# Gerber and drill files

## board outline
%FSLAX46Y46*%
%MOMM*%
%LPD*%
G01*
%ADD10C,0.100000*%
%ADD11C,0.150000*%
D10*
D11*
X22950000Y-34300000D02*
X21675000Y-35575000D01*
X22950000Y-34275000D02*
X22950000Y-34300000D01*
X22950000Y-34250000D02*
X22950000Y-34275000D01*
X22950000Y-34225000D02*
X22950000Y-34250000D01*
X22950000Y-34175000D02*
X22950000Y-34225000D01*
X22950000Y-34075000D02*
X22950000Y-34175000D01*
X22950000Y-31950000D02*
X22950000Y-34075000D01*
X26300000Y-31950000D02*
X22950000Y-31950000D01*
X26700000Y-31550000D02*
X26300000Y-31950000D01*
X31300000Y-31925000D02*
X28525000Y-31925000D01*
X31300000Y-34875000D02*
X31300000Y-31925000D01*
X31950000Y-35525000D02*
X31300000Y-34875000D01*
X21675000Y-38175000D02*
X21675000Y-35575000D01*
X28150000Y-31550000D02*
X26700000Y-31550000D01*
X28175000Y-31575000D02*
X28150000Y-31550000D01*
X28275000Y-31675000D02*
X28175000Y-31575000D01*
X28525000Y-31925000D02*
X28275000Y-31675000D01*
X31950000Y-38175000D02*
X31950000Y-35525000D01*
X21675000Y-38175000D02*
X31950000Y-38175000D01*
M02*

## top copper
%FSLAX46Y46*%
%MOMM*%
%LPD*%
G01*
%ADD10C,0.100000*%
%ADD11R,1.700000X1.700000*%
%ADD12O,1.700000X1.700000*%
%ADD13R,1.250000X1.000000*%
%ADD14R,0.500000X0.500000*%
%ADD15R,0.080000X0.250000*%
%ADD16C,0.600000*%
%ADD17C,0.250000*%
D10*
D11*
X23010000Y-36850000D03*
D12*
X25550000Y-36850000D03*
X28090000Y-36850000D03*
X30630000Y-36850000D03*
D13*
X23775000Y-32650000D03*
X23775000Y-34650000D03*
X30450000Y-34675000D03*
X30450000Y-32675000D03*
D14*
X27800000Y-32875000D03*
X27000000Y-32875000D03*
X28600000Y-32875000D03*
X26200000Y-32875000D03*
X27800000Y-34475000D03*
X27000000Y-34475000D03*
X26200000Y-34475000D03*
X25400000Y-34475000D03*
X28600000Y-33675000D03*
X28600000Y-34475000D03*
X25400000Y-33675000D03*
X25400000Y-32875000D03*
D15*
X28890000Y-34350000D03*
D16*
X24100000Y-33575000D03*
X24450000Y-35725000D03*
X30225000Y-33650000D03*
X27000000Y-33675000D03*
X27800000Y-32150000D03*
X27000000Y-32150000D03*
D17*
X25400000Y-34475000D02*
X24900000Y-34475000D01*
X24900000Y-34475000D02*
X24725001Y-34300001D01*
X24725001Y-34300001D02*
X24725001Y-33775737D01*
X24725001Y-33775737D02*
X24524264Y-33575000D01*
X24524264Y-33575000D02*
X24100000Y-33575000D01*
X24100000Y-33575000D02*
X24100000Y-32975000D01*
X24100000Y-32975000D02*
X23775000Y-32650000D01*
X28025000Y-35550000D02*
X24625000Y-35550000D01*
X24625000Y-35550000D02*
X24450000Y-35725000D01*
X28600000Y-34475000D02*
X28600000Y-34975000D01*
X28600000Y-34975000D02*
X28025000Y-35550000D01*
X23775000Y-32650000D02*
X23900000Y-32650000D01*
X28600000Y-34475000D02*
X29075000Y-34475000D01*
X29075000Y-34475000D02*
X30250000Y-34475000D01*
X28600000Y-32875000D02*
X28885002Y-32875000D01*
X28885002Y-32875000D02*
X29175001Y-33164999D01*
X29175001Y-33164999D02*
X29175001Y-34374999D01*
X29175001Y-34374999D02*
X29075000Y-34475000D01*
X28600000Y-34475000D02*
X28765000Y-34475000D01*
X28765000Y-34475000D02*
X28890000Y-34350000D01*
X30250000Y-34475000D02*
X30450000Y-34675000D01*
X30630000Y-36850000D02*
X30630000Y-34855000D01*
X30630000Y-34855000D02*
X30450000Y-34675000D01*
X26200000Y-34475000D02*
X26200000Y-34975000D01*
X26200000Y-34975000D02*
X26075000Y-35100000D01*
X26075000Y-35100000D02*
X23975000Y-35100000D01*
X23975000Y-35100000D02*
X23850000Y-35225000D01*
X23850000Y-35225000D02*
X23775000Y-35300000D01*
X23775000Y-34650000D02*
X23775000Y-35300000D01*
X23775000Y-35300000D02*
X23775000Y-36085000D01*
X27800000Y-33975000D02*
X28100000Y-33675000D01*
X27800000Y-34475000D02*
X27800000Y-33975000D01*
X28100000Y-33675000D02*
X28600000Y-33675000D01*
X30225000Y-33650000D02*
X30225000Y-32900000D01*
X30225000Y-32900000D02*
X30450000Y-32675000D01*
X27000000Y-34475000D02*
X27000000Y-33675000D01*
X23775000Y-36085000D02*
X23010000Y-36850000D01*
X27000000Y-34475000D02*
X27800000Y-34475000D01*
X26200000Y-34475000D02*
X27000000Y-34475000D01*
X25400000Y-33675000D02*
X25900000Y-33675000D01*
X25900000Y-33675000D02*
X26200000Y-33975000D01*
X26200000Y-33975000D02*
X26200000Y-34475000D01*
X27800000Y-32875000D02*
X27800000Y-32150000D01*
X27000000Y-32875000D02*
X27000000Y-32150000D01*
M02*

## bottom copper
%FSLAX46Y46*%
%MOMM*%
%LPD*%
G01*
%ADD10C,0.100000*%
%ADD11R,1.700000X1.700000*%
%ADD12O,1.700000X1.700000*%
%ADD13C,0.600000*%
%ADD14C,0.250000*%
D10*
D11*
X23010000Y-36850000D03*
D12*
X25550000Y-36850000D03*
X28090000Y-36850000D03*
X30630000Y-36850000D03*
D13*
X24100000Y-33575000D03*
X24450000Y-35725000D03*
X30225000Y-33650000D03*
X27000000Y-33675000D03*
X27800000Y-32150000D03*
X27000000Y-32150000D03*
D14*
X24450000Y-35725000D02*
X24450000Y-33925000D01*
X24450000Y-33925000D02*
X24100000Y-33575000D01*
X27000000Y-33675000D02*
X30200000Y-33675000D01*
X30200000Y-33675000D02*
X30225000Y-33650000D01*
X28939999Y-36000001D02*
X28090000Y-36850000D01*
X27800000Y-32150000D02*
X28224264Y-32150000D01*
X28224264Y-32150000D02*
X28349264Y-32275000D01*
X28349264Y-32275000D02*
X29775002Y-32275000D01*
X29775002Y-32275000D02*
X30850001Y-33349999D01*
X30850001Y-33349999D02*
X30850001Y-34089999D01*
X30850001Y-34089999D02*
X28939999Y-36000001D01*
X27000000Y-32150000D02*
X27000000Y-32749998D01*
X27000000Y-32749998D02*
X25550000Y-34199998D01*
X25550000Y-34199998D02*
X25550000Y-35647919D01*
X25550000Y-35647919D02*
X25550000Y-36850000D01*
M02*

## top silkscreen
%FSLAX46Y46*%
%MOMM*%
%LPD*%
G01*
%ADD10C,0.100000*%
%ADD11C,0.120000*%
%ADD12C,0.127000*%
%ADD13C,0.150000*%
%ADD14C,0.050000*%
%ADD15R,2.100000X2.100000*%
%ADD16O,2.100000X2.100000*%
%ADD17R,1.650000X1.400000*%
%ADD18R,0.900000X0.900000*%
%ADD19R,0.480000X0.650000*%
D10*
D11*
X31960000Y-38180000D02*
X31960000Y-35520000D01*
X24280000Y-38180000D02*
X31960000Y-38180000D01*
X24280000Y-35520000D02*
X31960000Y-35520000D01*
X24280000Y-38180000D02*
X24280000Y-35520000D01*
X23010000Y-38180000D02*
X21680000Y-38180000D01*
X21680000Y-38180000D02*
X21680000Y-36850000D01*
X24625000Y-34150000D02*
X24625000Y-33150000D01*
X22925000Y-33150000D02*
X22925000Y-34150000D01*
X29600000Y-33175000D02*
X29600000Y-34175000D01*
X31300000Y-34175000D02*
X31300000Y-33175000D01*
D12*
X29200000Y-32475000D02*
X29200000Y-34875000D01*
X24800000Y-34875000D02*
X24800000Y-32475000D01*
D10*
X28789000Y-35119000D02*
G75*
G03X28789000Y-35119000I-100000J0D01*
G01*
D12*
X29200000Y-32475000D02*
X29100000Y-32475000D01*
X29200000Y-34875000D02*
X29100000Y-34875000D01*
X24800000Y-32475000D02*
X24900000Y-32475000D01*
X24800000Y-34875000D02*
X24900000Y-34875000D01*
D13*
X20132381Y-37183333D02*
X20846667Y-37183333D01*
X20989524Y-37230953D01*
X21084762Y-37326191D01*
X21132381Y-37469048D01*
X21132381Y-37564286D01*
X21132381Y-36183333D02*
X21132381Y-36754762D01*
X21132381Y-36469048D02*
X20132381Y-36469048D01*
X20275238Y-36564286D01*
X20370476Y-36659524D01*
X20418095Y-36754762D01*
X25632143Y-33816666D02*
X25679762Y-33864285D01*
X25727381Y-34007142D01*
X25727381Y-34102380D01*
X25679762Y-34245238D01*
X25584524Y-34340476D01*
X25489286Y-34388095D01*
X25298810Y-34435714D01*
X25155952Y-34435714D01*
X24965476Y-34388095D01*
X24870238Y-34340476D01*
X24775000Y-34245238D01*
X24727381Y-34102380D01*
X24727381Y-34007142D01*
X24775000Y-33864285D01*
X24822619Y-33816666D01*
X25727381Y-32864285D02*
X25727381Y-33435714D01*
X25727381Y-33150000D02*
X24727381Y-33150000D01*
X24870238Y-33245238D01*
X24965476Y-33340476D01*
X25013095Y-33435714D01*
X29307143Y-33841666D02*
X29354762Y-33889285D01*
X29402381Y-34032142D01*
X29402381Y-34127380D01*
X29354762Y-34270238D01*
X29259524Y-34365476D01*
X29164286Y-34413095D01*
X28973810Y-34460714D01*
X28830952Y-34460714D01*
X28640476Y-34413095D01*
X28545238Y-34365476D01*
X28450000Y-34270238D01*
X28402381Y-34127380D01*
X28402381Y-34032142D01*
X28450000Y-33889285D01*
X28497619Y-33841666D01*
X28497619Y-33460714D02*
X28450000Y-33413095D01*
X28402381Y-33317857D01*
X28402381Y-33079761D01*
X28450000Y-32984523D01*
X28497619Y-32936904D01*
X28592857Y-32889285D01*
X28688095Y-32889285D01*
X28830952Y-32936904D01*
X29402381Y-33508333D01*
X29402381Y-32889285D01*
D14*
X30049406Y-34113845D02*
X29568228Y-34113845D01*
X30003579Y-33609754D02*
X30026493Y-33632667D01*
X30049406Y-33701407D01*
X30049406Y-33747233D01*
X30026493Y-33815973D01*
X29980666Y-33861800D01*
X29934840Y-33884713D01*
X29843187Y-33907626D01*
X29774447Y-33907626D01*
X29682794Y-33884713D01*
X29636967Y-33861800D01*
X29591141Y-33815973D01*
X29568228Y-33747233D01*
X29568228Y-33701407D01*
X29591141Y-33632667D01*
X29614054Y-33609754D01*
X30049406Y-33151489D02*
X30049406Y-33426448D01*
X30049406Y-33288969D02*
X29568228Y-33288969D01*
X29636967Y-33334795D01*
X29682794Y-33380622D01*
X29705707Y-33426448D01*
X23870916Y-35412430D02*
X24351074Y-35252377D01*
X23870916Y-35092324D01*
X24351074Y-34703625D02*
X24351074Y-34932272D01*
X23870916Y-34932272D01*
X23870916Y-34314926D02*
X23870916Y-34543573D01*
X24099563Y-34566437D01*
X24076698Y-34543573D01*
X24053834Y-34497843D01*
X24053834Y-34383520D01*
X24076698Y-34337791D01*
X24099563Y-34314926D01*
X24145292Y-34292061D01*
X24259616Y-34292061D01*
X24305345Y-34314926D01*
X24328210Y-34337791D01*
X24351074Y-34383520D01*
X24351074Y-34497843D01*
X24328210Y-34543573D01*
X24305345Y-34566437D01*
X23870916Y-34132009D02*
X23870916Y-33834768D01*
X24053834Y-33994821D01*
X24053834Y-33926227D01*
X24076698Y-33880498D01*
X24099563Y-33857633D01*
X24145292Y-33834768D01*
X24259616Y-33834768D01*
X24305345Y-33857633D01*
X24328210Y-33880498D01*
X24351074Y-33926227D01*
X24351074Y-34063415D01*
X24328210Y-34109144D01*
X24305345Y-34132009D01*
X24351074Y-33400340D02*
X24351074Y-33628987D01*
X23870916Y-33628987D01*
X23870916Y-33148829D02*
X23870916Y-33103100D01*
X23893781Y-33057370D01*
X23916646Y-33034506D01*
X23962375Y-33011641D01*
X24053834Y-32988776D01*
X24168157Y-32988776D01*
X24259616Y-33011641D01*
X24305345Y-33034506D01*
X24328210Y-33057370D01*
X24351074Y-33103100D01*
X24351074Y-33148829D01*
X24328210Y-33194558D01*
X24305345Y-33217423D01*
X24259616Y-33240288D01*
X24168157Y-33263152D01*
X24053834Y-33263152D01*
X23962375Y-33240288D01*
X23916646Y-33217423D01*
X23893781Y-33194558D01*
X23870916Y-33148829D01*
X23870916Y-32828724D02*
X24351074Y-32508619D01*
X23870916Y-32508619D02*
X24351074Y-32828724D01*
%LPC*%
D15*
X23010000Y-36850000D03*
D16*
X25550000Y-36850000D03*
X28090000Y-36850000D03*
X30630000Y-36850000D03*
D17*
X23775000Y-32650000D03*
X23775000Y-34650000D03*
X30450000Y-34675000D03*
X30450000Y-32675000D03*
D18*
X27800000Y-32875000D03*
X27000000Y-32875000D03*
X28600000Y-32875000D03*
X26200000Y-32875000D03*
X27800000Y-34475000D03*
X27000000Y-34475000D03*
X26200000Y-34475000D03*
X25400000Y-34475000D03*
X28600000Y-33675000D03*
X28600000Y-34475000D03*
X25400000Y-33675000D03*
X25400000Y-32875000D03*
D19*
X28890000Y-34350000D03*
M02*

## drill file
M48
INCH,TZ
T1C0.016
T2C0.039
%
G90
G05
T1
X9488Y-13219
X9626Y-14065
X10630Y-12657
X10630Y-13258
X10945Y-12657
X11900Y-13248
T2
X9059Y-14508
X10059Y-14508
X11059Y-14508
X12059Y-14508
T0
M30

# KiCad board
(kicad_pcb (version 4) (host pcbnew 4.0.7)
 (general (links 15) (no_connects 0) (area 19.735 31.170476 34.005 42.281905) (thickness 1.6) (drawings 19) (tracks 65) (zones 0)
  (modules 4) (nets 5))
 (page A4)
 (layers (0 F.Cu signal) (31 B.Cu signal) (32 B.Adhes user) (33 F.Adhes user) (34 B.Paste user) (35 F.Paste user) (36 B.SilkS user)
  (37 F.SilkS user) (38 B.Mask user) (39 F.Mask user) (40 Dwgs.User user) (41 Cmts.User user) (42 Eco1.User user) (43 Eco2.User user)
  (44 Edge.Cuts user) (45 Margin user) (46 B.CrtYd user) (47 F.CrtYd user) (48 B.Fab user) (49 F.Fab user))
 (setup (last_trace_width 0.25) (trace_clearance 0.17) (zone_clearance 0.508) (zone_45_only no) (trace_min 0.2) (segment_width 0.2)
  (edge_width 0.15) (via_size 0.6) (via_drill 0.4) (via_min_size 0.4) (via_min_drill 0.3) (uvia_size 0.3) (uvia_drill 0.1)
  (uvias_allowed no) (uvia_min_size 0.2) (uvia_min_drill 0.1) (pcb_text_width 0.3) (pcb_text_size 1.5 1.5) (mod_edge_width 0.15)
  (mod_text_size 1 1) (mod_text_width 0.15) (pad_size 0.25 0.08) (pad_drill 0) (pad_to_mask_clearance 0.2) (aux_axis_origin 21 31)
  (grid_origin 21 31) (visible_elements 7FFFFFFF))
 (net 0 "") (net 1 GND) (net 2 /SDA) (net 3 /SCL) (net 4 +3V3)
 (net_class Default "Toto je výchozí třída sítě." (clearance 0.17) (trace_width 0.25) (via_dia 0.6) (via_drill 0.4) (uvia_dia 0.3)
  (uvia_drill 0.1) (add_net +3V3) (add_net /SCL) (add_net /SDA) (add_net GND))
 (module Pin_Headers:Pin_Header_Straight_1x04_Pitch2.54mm (layer F.Cu) (at 23.01 36.85 90)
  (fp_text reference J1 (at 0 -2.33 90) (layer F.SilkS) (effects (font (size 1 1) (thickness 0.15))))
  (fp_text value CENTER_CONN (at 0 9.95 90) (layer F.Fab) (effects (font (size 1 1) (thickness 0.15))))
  (fp_line (start -1.33 8.95) (end 1.33 8.95) (layer F.SilkS) (width 0.12))
  (fp_line (start -1.33 1.27) (end -1.33 8.95) (layer F.SilkS) (width 0.12))
  (fp_line (start 1.33 1.27) (end 1.33 8.95) (layer F.SilkS) (width 0.12))
  (fp_line (start -1.33 1.27) (end 1.33 1.27) (layer F.SilkS) (width 0.12))
  (fp_line (start -1.33 0) (end -1.33 -1.33) (layer F.SilkS) (width 0.12))
  (fp_line (start -1.33 -1.33) (end 0 -1.33) (layer F.SilkS) (width 0.12))
  (pad 1 thru_hole rect (at 0 0 90) (size 1.7 1.7) (drill 1) (layers *.Cu *.Mask) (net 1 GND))
  (pad 2 thru_hole oval (at 0 2.54 90) (size 1.7 1.7) (drill 1) (layers *.Cu *.Mask) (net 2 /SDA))
  (pad 3 thru_hole oval (at 0 5.08 90) (size 1.7 1.7) (drill 1) (layers *.Cu *.Mask) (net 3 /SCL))
  (pad 4 thru_hole oval (at 0 7.62 90) (size 1.7 1.7) (drill 1) (layers *.Cu *.Mask) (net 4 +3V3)))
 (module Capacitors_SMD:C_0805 (layer F.Cu) (at 23.775 33.65 270)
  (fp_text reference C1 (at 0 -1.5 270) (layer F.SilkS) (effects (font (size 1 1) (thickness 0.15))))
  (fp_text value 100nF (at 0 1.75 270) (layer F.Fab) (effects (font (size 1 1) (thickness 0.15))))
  (fp_line (start 0.5 -0.85) (end -0.5 -0.85) (layer F.SilkS) (width 0.12))
  (fp_line (start -0.5 0.85) (end 0.5 0.85) (layer F.SilkS) (width 0.12))
  (pad 1 smd rect (at -1 0 270) (size 1 1.25) (layers F.Cu F.Paste F.Mask) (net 4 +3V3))
  (pad 2 smd rect (at 1 0 270) (size 1 1.25) (layers F.Cu F.Paste F.Mask) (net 1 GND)))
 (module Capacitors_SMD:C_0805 (layer F.Cu) (at 30.45 33.675 90)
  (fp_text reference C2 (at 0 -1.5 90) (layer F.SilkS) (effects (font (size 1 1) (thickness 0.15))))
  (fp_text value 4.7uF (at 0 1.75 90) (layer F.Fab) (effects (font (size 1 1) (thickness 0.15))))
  (fp_line (start 0.5 -0.85) (end -0.5 -0.85) (layer F.SilkS) (width 0.12))
  (fp_line (start -0.5 0.85) (end 0.5 0.85) (layer F.SilkS) (width 0.12))
  (pad 1 smd rect (at -1 0 90) (size 1 1.25) (layers F.Cu F.Paste F.Mask) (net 4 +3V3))
  (pad 2 smd rect (at 1 0 90) (size 1 1.25) (layers F.Cu F.Paste F.Mask) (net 1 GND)))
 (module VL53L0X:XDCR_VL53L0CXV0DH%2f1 (layer F.Cu) (at 27 33.675 270)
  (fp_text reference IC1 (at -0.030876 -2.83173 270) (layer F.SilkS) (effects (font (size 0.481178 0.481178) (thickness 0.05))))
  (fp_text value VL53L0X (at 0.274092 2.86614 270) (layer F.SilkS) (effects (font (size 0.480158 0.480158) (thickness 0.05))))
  (fp_line (start -1.2 -2.2) (end 1.2 -2.2) (layer F.SilkS) (width 0.127))
  (fp_line (start 1.2 2.2) (end -1.2 2.2) (layer F.SilkS) (width 0.127))
  (fp_circle (center 1.444 -1.689) (end 1.544 -1.689) (layer F.SilkS) (width 0))
  (fp_line (start -1.2 -2.2) (end -1.2 -2.1) (layer F.SilkS) (width 0.127))
  (fp_line (start 1.2 -2.2) (end 1.2 -2.1) (layer F.SilkS) (width 0.127))
  (fp_line (start -1.2 2.2) (end -1.2 2.1) (layer F.SilkS) (width 0.127))
  (fp_line (start 1.2 2.2) (end 1.2 2.1) (layer F.SilkS) (width 0.127))
  (pad 10 smd rect (at -0.8 -0.8 270) (size 0.5 0.5) (layers F.Cu F.Paste F.Mask) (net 3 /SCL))
  (pad 9 smd rect (at -0.8 0 270) (size 0.5 0.5) (layers F.Cu F.Paste F.Mask) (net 2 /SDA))
  (pad 11 smd rect (at -0.8 -1.6 270) (size 0.5 0.5) (layers F.Cu F.Paste F.Mask) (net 4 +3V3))
  (pad 8 smd rect (at -0.8 0.8 270) (size 0.5 0.5) (layers F.Cu F.Paste F.Mask))
  (pad 2 smd rect (at 0.8 -0.8 270) (size 0.5 0.5) (layers F.Cu F.Paste F.Mask) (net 1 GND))
  (pad 3 smd rect (at 0.8 0 270) (size 0.5 0.5) (layers F.Cu F.Paste F.Mask) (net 1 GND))
  (pad 4 smd rect (at 0.8 0.8 270) (size 0.5 0.5) (layers F.Cu F.Paste F.Mask) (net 1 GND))
  (pad 5 smd rect (at 0.8 1.6 270) (size 0.5 0.5) (layers F.Cu F.Paste F.Mask) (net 4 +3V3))
  (pad 12 smd rect (at 0 -1.6 270) (size 0.5 0.5) (layers F.Cu F.Paste F.Mask) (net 1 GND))
  (pad 1 smd rect (at 0.8 -1.6 270) (size 0.5 0.5) (layers F.Cu F.Paste F.Mask) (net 4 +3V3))
  (pad 6 smd rect (at 0 1.6 270) (size 0.5 0.5) (layers F.Cu F.Paste F.Mask) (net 1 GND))
  (pad 7 smd rect (at -0.8 1.6 270) (size 0.5 0.5) (layers F.Cu F.Paste F.Mask))
  (pad 1.1 smd rect (at 0.675 -1.89 270) (size 0.25 0.08) (layers F.Cu F.Paste F.Mask) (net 4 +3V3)))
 (gr_line (start 22.95 34.3) (end 21.675 35.575) (angle 90) (layer Edge.Cuts) (width 0.15))
 (gr_line (start 22.95 34.275) (end 22.95 34.3) (angle 90) (layer Edge.Cuts) (width 0.15))
 (gr_line (start 22.95 34.25) (end 22.95 34.275) (angle 90) (layer Edge.Cuts) (width 0.15))
 (gr_line (start 22.95 34.225) (end 22.95 34.25) (angle 90) (layer Edge.Cuts) (width 0.15))
 (gr_line (start 22.95 34.175) (end 22.95 34.225) (angle 90) (layer Edge.Cuts) (width 0.15))
 (gr_line (start 22.95 34.075) (end 22.95 34.175) (angle 90) (layer Edge.Cuts) (width 0.15))
 (gr_line (start 22.95 31.95) (end 22.95 34.075) (angle 90) (layer Edge.Cuts) (width 0.15))
 (gr_line (start 26.3 31.95) (end 22.95 31.95) (angle 90) (layer Edge.Cuts) (width 0.15))
 (gr_line (start 26.7 31.55) (end 26.3 31.95) (angle 90) (layer Edge.Cuts) (width 0.15))
 (gr_line (start 31.3 31.925) (end 28.525 31.925) (angle 90) (layer Edge.Cuts) (width 0.15))
 (gr_line (start 31.3 34.875) (end 31.3 31.925) (angle 90) (layer Edge.Cuts) (width 0.15))
 (gr_line (start 31.95 35.525) (end 31.3 34.875) (angle 90) (layer Edge.Cuts) (width 0.15))
 (gr_line (start 21.675 38.175) (end 21.675 35.575) (layer Edge.Cuts) (width 0.15))
 (gr_line (start 28.15 31.55) (end 26.7 31.55) (layer Edge.Cuts) (width 0.15))
 (gr_line (start 28.175 31.575) (end 28.15 31.55) (layer Edge.Cuts) (width 0.15))
 (gr_line (start 28.275 31.675) (end 28.175 31.575) (layer Edge.Cuts) (width 0.15))
 (gr_line (start 28.525 31.925) (end 28.275 31.675) (layer Edge.Cuts) (width 0.15))
 (gr_line (start 31.95 38.175) (end 31.95 35.525) (layer Edge.Cuts) (width 0.15))
 (gr_line (start 21.675 38.175) (end 31.95 38.175) (layer Edge.Cuts) (width 0.15))
 (segment (start 25.4 34.475) (end 24.9 34.475) (width 0.25) (layer F.Cu) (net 4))
 (segment (start 24.9 34.475) (end 24.725001 34.300001) (width 0.25) (layer F.Cu) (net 4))
 (segment (start 24.725001 34.300001) (end 24.725001 33.775737) (width 0.25) (layer F.Cu) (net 4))
 (segment (start 24.725001 33.775737) (end 24.524264 33.575) (width 0.25) (layer F.Cu) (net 4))
 (segment (start 24.524264 33.575) (end 24.1 33.575) (width 0.25) (layer F.Cu) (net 4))
 (segment (start 24.1 33.575) (end 24.1 32.975) (width 0.25) (layer F.Cu) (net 4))
 (segment (start 24.1 32.975) (end 23.775 32.65) (width 0.25) (layer F.Cu) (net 4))
 (segment (start 24.45 35.725) (end 24.45 33.925) (width 0.25) (layer B.Cu) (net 4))
 (segment (start 24.45 33.925) (end 24.1 33.575) (width 0.25) (layer B.Cu) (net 4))
 (via (at 24.1 33.575) (size 0.6) (drill 0.4) (layers F.Cu B.Cu) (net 4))
 (segment (start 28.025 35.55) (end 24.625 35.55) (width 0.25) (layer F.Cu) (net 4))
 (segment (start 24.625 35.55) (end 24.45 35.725) (width 0.25) (layer F.Cu) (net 4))
 (via (at 24.45 35.725) (size 0.6) (drill 0.4) (layers F.Cu B.Cu) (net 4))
 (segment (start 28.6 34.475) (end 28.6 34.975) (width 0.25) (layer F.Cu) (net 4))
 (segment (start 28.6 34.975) (end 28.025 35.55) (width 0.25) (layer F.Cu) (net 4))
 (segment (start 23.775 32.65) (end 23.9 32.65) (width 0.25) (layer F.Cu) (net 4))
 (segment (start 28.6 34.475) (end 29.075 34.475) (width 0.25) (layer F.Cu) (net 4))
 (segment (start 29.075 34.475) (end 30.25 34.475) (width 0.25) (layer F.Cu) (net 4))
 (segment (start 28.6 32.875) (end 28.885002 32.875) (width 0.25) (layer F.Cu) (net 4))
 (segment (start 28.885002 32.875) (end 29.175001 33.164999) (width 0.25) (layer F.Cu) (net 4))
 (segment (start 29.175001 33.164999) (end 29.175001 34.374999) (width 0.25) (layer F.Cu) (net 4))
 (segment (start 29.175001 34.374999) (end 29.075 34.475) (width 0.25) (layer F.Cu) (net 4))
 (segment (start 28.6 34.475) (end 28.765 34.475) (width 0.25) (layer F.Cu) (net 4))
 (segment (start 28.765 34.475) (end 28.89 34.35) (width 0.25) (layer F.Cu) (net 4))
 (segment (start 30.25 34.475) (end 30.45 34.675) (width 0.25) (layer F.Cu) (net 4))
 (segment (start 30.63 36.85) (end 30.63 34.855) (width 0.25) (layer F.Cu) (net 4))
 (segment (start 30.63 34.855) (end 30.45 34.675) (width 0.25) (layer F.Cu) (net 4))
 (segment (start 26.2 34.475) (end 26.2 34.975) (width 0.25) (layer F.Cu) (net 1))
 (segment (start 26.2 34.975) (end 26.075 35.1) (width 0.25) (layer F.Cu) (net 1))
 (segment (start 26.075 35.1) (end 23.975 35.1) (width 0.25) (layer F.Cu) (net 1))
 (segment (start 23.975 35.1) (end 23.85 35.225) (width 0.25) (layer F.Cu) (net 1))
 (segment (start 23.85 35.225) (end 23.775 35.3) (width 0.25) (layer F.Cu) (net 1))
 (segment (start 23.775 34.65) (end 23.775 35.3) (width 0.25) (layer F.Cu) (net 1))
 (segment (start 23.775 35.3) (end 23.775 36.085) (width 0.25) (layer F.Cu) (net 1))
 (segment (start 27.8 33.975) (end 28.1 33.675) (width 0.25) (layer F.Cu) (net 1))
 (segment (start 27.8 34.475) (end 27.8 33.975) (width 0.25) (layer F.Cu) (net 1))
 (segment (start 28.1 33.675) (end 28.6 33.675) (width 0.25) (layer F.Cu) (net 1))
 (segment (start 27 33.675) (end 30.2 33.675) (width 0.25) (layer B.Cu) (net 1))
 (segment (start 30.225 33.65) (end 30.225 32.9) (width 0.25) (layer F.Cu) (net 1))
 (segment (start 30.225 32.9) (end 30.45 32.675) (width 0.25) (layer F.Cu) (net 1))
 (segment (start 30.2 33.675) (end 30.225 33.65) (width 0.25) (layer B.Cu) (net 1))
 (via (at 30.225 33.65) (size 0.6) (drill 0.4) (layers F.Cu B.Cu) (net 1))
 (segment (start 27 34.475) (end 27 33.675) (width 0.25) (layer F.Cu) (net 1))
 (via (at 27 33.675) (size 0.6) (drill 0.4) (layers F.Cu B.Cu) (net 1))
 (segment (start 23.775 36.085) (end 23.01 36.85) (width 0.25) (layer F.Cu) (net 1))
 (segment (start 27 34.475) (end 27.8 34.475) (width 0.25) (layer F.Cu) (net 1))
 (segment (start 26.2 34.475) (end 27 34.475) (width 0.25) (layer F.Cu) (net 1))
 (segment (start 25.4 33.675) (end 25.9 33.675) (width 0.25) (layer F.Cu) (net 1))
 (segment (start 25.9 33.675) (end 26.2 33.975) (width 0.25) (layer F.Cu) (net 1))
 (segment (start 26.2 33.975) (end 26.2 34.475) (width 0.25) (layer F.Cu) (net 1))
 (segment (start 28.939999 36.000001) (end 28.09 36.85) (width 0.25) (layer B.Cu) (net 3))
 (segment (start 27.8 32.15) (end 28.224264 32.15) (width 0.25) (layer B.Cu) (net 3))
 (segment (start 28.224264 32.15) (end 28.349264 32.275) (width 0.25) (layer B.Cu) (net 3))
 (segment (start 28.349264 32.275) (end 29.775002 32.275) (width 0.25) (layer B.Cu) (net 3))
 (segment (start 27.8 32.875) (end 27.8 32.15) (width 0.25) (layer F.Cu) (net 3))
 (via (at 27.8 32.15) (size 0.6) (drill 0.4) (layers F.Cu B.Cu) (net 3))
 (segment (start 29.775002 32.275) (end 30.850001 33.349999) (width 0.25) (layer B.Cu) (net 3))
 (segment (start 30.850001 33.349999) (end 30.850001 34.089999) (width 0.25) (layer B.Cu) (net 3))
 (segment (start 30.850001 34.089999) (end 28.939999 36.000001) (width 0.25) (layer B.Cu) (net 3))
 (segment (start 27 32.15) (end 27 32.749998) (width 0.25) (layer B.Cu) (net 2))
 (segment (start 27 32.749998) (end 25.55 34.199998) (width 0.25) (layer B.Cu) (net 2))
 (segment (start 25.55 34.199998) (end 25.55 35.647919) (width 0.25) (layer B.Cu) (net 2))
 (segment (start 25.55 35.647919) (end 25.55 36.85) (width 0.25) (layer B.Cu) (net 2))
 (segment (start 27 32.875) (end 27 32.15) (width 0.25) (layer F.Cu) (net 2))
 (via (at 27 32.15) (size 0.6) (drill 0.4) (layers F.Cu B.Cu) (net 2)))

